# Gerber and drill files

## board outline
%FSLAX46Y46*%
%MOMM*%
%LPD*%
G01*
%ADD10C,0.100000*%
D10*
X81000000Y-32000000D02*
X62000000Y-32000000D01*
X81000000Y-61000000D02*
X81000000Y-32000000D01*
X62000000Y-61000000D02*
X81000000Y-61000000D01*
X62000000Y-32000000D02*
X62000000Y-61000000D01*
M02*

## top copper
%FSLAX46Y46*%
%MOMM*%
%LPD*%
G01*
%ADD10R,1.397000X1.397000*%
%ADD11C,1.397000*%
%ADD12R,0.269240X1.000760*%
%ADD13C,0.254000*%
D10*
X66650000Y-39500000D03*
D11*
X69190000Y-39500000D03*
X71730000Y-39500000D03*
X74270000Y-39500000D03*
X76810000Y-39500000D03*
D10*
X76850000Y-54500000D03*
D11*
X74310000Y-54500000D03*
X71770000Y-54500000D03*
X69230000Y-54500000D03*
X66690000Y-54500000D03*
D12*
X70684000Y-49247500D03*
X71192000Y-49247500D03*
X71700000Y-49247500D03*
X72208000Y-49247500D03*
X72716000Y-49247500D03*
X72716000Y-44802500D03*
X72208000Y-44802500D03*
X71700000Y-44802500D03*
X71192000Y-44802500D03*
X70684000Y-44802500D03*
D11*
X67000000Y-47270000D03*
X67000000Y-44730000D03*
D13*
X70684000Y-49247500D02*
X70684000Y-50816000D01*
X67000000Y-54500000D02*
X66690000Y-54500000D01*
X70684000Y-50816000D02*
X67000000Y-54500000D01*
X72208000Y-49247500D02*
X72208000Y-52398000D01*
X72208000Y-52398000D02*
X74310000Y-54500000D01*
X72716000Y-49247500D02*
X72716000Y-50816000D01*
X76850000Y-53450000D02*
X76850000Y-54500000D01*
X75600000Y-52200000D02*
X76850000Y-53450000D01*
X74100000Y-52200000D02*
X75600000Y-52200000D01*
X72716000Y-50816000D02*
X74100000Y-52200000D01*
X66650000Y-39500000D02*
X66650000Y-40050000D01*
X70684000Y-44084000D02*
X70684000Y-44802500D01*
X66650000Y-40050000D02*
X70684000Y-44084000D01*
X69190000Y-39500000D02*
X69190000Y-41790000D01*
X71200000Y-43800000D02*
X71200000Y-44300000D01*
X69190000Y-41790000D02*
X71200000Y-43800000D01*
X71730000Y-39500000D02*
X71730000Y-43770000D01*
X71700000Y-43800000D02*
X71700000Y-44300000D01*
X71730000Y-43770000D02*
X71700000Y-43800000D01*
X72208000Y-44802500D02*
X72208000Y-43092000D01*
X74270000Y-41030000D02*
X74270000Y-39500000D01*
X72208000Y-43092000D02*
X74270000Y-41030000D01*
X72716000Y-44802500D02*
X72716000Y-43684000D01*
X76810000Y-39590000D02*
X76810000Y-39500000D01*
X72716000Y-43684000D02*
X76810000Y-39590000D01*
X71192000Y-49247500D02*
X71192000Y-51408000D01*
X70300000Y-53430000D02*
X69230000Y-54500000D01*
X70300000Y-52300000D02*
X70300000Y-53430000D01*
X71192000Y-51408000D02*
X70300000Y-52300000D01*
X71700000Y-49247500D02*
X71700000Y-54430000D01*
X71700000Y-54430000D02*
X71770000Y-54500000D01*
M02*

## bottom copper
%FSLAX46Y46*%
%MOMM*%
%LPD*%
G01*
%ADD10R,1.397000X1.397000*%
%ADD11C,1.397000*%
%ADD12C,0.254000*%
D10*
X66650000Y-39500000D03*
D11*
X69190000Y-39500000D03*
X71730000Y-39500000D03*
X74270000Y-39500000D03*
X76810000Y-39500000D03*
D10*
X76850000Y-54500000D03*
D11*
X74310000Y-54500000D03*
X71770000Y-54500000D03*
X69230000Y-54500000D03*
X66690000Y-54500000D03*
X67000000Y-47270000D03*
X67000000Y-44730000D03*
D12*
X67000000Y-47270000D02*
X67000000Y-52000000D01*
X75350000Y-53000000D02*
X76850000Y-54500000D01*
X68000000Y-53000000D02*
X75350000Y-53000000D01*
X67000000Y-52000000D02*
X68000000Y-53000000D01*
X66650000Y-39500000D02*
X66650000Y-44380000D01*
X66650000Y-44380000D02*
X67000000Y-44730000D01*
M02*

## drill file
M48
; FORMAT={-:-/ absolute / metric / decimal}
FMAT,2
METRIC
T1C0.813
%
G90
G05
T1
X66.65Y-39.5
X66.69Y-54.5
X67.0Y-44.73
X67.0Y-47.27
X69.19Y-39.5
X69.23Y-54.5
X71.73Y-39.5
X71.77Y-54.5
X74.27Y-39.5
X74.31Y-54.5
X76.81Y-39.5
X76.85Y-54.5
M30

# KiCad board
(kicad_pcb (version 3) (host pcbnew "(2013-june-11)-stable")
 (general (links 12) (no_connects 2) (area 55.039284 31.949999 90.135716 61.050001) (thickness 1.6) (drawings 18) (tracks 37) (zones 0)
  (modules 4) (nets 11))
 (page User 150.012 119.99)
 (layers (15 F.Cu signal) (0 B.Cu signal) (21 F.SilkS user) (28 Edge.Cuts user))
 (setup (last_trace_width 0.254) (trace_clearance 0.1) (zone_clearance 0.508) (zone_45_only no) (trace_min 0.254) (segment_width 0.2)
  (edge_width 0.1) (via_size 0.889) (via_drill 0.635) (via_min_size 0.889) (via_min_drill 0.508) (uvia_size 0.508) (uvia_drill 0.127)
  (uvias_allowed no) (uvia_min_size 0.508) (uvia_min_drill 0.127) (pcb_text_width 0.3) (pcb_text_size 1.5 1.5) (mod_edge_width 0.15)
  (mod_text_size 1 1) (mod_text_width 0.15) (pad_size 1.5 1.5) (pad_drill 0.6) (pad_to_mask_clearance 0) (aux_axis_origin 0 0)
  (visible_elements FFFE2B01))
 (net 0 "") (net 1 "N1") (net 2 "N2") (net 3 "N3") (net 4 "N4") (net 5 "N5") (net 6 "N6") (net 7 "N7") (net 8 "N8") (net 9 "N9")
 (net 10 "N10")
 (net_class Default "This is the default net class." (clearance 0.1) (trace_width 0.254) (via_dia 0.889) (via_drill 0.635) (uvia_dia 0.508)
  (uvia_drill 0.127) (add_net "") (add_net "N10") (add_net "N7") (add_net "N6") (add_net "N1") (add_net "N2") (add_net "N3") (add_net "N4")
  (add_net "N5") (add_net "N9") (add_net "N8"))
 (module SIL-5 (layer F.Cu) (at 73 39.5)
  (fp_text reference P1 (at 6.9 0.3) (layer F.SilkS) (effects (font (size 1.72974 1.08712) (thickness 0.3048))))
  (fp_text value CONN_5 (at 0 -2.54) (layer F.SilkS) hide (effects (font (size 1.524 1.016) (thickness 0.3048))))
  (pad 1 thru_hole rect (at -6.35 0) (size 1.397 1.397) (drill 0.8128) (layers *.Cu *.Mask) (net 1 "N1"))
  (pad 2 thru_hole circle (at -3.81 0) (size 1.397 1.397) (drill 0.8128) (layers *.Cu *.Mask) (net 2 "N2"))
  (pad 3 thru_hole circle (at -1.27 0) (size 1.397 1.397) (drill 0.8128) (layers *.Cu *.Mask) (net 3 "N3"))
  (pad 4 thru_hole circle (at 1.27 0) (size 1.397 1.397) (drill 0.8128) (layers *.Cu *.Mask) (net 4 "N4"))
  (pad 5 thru_hole circle (at 3.81 0) (size 1.397 1.397) (drill 0.8128) (layers *.Cu *.Mask) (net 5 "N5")))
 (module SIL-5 (layer F.Cu) (at 70.5 54.5 180)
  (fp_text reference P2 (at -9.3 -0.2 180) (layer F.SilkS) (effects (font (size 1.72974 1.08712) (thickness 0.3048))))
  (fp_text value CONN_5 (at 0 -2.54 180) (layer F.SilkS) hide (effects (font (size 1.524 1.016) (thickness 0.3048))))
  (pad 1 thru_hole rect (at -6.35 0 180) (size 1.397 1.397) (drill 0.8128) (layers *.Cu *.Mask) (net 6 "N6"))
  (pad 2 thru_hole circle (at -3.81 0 180) (size 1.397 1.397) (drill 0.8128) (layers *.Cu *.Mask) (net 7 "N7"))
  (pad 3 thru_hole circle (at -1.27 0 180) (size 1.397 1.397) (drill 0.8128) (layers *.Cu *.Mask) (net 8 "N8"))
  (pad 4 thru_hole circle (at 1.27 0 180) (size 1.397 1.397) (drill 0.8128) (layers *.Cu *.Mask) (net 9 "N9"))
  (pad 5 thru_hole circle (at 3.81 0 180) (size 1.397 1.397) (drill 0.8128) (layers *.Cu *.Mask) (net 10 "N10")))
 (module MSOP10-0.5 (layer F.Cu) (at 71.7 47.025)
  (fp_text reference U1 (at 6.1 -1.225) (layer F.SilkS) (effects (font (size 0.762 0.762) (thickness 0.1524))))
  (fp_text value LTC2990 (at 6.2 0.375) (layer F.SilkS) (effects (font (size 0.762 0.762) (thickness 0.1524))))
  (pad 1 smd rect (at -1.016 2.2225) (size 0.26924 1.00076) (layers F.Cu) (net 10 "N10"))
  (pad 2 smd rect (at -0.508 2.2225) (size 0.26924 1.00076) (layers F.Cu) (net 9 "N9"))
  (pad 3 smd rect (at 0 2.2225) (size 0.26924 1.00076) (layers F.Cu) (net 8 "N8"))
  (pad 4 smd rect (at 0.508 2.2225) (size 0.26924 1.00076) (layers F.Cu) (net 7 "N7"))
  (pad 5 smd rect (at 1.016 2.2225) (size 0.26924 1.00076) (layers F.Cu) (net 6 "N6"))
  (pad 6 smd rect (at 1.016 -2.2225) (size 0.26924 1.00076) (layers F.Cu) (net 5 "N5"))
  (pad 7 smd rect (at 0.508 -2.2225) (size 0.26924 1.00076) (layers F.Cu) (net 4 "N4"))
  (pad 8 smd rect (at 0 -2.2225) (size 0.26924 1.00076) (layers F.Cu) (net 3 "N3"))
  (pad 9 smd rect (at -0.508 -2.2225) (size 0.26924 1.00076) (layers F.Cu) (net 2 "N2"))
  (pad 10 smd rect (at -1.016 -2.2225) (size 0.26924 1.00076) (layers F.Cu) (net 1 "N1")))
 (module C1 (layer F.Cu) (at 67 46 90)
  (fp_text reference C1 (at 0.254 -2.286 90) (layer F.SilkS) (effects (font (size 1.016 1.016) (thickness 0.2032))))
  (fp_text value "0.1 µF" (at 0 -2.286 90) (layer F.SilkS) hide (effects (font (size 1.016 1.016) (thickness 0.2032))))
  (pad 1 thru_hole circle (at -1.27 0 90) (size 1.397 1.397) (drill 0.8128) (layers *.Cu *.Mask F.SilkS) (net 6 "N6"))
  (pad 2 thru_hole circle (at 1.27 0 90) (size 1.397 1.397) (drill 0.8128) (layers *.Cu *.Mask F.SilkS) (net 1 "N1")))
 (gr_line (start 81 32) (end 62 32) (angle 90) (layer Edge.Cuts) (width 0.1))
 (gr_line (start 81 61) (end 81 32) (angle 90) (layer Edge.Cuts) (width 0.1))
 (gr_line (start 62 61) (end 81 61) (angle 90) (layer Edge.Cuts) (width 0.1))
 (gr_line (start 62 32) (end 62 61) (angle 90) (layer Edge.Cuts) (width 0.1))
 (segment (start 70.684 49.2475) (end 70.684 50.816) (width 0.254) (layer F.Cu) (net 10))
 (segment (start 67 54.5) (end 66.69 54.5) (width 0.254) (layer F.Cu) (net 10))
 (segment (start 70.684 50.816) (end 67 54.5) (width 0.254) (layer F.Cu) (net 10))
 (segment (start 72.208 49.2475) (end 72.208 52.398) (width 0.254) (layer F.Cu) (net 7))
 (segment (start 72.208 52.398) (end 74.31 54.5) (width 0.254) (layer F.Cu) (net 7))
 (segment (start 67 47.27) (end 67 52) (width 0.254) (layer B.Cu) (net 6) (status 10))
 (segment (start 75.35 53) (end 76.85 54.5) (width 0.254) (layer B.Cu) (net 6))
 (segment (start 68 53) (end 75.35 53) (width 0.254) (layer B.Cu) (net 6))
 (segment (start 67 52) (end 68 53) (width 0.254) (layer B.Cu) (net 6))
 (segment (start 72.716 49.2475) (end 72.716 50.816) (width 0.254) (layer F.Cu) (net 6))
 (segment (start 76.85 53.45) (end 76.85 54.5) (width 0.254) (layer F.Cu) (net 6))
 (segment (start 75.6 52.2) (end 76.85 53.45) (width 0.254) (layer F.Cu) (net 6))
 (segment (start 74.1 52.2) (end 75.6 52.2) (width 0.254) (layer F.Cu) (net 6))
 (segment (start 72.716 50.816) (end 74.1 52.2) (width 0.254) (layer F.Cu) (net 6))
 (segment (start 66.65 39.5) (end 66.65 44.38) (width 0.254) (layer B.Cu) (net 1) (status 20))
 (segment (start 66.65 44.38) (end 67 44.73) (width 0.254) (layer B.Cu) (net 1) (status 30))
 (segment (start 66.65 39.5) (end 66.65 40.05) (width 0.254) (layer F.Cu) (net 1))
 (segment (start 70.684 44.084) (end 70.684 44.8025) (width 0.254) (layer F.Cu) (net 1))
 (segment (start 66.65 40.05) (end 70.684 44.084) (width 0.254) (layer F.Cu) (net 1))
 (segment (start 69.19 39.5) (end 69.19 41.79) (width 0.254) (layer F.Cu) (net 2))
 (segment (start 71.2 43.8) (end 71.2 44.3) (width 0.254) (layer F.Cu) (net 2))
 (segment (start 69.19 41.79) (end 71.2 43.8) (width 0.254) (layer F.Cu) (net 2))
 (segment (start 71.73 39.5) (end 71.73 43.77) (width 0.254) (layer F.Cu) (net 3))
 (segment (start 71.7 43.8) (end 71.7 44.3) (width 0.254) (layer F.Cu) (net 3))
 (segment (start 71.73 43.77) (end 71.7 43.8) (width 0.254) (layer F.Cu) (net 3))
 (segment (start 72.208 44.8025) (end 72.208 43.092) (width 0.254) (layer F.Cu) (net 4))
 (segment (start 74.27 41.03) (end 74.27 39.5) (width 0.254) (layer F.Cu) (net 4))
 (segment (start 72.208 43.092) (end 74.27 41.03) (width 0.254) (layer F.Cu) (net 4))
 (segment (start 72.716 44.8025) (end 72.716 43.684) (width 0.254) (layer F.Cu) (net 5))
 (segment (start 76.81 39.59) (end 76.81 39.5) (width 0.254) (layer F.Cu) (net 5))
 (segment (start 72.716 43.684) (end 76.81 39.59) (width 0.254) (layer F.Cu) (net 5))
 (segment (start 71.192 49.2475) (end 71.192 51.408) (width 0.254) (layer F.Cu) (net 9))
 (segment (start 70.3 53.43) (end 69.23 54.5) (width 0.254) (layer F.Cu) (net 9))
 (segment (start 70.3 52.3) (end 70.3 53.43) (width 0.254) (layer F.Cu) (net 9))
 (segment (start 71.192 51.408) (end 70.3 52.3) (width 0.254) (layer F.Cu) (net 9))
 (segment (start 71.7 49.2475) (end 71.7 54.43) (width 0.254) (layer F.Cu) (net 8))
 (segment (start 71.7 54.43) (end 71.77 54.5) (width 0.254) (layer F.Cu) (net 8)))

